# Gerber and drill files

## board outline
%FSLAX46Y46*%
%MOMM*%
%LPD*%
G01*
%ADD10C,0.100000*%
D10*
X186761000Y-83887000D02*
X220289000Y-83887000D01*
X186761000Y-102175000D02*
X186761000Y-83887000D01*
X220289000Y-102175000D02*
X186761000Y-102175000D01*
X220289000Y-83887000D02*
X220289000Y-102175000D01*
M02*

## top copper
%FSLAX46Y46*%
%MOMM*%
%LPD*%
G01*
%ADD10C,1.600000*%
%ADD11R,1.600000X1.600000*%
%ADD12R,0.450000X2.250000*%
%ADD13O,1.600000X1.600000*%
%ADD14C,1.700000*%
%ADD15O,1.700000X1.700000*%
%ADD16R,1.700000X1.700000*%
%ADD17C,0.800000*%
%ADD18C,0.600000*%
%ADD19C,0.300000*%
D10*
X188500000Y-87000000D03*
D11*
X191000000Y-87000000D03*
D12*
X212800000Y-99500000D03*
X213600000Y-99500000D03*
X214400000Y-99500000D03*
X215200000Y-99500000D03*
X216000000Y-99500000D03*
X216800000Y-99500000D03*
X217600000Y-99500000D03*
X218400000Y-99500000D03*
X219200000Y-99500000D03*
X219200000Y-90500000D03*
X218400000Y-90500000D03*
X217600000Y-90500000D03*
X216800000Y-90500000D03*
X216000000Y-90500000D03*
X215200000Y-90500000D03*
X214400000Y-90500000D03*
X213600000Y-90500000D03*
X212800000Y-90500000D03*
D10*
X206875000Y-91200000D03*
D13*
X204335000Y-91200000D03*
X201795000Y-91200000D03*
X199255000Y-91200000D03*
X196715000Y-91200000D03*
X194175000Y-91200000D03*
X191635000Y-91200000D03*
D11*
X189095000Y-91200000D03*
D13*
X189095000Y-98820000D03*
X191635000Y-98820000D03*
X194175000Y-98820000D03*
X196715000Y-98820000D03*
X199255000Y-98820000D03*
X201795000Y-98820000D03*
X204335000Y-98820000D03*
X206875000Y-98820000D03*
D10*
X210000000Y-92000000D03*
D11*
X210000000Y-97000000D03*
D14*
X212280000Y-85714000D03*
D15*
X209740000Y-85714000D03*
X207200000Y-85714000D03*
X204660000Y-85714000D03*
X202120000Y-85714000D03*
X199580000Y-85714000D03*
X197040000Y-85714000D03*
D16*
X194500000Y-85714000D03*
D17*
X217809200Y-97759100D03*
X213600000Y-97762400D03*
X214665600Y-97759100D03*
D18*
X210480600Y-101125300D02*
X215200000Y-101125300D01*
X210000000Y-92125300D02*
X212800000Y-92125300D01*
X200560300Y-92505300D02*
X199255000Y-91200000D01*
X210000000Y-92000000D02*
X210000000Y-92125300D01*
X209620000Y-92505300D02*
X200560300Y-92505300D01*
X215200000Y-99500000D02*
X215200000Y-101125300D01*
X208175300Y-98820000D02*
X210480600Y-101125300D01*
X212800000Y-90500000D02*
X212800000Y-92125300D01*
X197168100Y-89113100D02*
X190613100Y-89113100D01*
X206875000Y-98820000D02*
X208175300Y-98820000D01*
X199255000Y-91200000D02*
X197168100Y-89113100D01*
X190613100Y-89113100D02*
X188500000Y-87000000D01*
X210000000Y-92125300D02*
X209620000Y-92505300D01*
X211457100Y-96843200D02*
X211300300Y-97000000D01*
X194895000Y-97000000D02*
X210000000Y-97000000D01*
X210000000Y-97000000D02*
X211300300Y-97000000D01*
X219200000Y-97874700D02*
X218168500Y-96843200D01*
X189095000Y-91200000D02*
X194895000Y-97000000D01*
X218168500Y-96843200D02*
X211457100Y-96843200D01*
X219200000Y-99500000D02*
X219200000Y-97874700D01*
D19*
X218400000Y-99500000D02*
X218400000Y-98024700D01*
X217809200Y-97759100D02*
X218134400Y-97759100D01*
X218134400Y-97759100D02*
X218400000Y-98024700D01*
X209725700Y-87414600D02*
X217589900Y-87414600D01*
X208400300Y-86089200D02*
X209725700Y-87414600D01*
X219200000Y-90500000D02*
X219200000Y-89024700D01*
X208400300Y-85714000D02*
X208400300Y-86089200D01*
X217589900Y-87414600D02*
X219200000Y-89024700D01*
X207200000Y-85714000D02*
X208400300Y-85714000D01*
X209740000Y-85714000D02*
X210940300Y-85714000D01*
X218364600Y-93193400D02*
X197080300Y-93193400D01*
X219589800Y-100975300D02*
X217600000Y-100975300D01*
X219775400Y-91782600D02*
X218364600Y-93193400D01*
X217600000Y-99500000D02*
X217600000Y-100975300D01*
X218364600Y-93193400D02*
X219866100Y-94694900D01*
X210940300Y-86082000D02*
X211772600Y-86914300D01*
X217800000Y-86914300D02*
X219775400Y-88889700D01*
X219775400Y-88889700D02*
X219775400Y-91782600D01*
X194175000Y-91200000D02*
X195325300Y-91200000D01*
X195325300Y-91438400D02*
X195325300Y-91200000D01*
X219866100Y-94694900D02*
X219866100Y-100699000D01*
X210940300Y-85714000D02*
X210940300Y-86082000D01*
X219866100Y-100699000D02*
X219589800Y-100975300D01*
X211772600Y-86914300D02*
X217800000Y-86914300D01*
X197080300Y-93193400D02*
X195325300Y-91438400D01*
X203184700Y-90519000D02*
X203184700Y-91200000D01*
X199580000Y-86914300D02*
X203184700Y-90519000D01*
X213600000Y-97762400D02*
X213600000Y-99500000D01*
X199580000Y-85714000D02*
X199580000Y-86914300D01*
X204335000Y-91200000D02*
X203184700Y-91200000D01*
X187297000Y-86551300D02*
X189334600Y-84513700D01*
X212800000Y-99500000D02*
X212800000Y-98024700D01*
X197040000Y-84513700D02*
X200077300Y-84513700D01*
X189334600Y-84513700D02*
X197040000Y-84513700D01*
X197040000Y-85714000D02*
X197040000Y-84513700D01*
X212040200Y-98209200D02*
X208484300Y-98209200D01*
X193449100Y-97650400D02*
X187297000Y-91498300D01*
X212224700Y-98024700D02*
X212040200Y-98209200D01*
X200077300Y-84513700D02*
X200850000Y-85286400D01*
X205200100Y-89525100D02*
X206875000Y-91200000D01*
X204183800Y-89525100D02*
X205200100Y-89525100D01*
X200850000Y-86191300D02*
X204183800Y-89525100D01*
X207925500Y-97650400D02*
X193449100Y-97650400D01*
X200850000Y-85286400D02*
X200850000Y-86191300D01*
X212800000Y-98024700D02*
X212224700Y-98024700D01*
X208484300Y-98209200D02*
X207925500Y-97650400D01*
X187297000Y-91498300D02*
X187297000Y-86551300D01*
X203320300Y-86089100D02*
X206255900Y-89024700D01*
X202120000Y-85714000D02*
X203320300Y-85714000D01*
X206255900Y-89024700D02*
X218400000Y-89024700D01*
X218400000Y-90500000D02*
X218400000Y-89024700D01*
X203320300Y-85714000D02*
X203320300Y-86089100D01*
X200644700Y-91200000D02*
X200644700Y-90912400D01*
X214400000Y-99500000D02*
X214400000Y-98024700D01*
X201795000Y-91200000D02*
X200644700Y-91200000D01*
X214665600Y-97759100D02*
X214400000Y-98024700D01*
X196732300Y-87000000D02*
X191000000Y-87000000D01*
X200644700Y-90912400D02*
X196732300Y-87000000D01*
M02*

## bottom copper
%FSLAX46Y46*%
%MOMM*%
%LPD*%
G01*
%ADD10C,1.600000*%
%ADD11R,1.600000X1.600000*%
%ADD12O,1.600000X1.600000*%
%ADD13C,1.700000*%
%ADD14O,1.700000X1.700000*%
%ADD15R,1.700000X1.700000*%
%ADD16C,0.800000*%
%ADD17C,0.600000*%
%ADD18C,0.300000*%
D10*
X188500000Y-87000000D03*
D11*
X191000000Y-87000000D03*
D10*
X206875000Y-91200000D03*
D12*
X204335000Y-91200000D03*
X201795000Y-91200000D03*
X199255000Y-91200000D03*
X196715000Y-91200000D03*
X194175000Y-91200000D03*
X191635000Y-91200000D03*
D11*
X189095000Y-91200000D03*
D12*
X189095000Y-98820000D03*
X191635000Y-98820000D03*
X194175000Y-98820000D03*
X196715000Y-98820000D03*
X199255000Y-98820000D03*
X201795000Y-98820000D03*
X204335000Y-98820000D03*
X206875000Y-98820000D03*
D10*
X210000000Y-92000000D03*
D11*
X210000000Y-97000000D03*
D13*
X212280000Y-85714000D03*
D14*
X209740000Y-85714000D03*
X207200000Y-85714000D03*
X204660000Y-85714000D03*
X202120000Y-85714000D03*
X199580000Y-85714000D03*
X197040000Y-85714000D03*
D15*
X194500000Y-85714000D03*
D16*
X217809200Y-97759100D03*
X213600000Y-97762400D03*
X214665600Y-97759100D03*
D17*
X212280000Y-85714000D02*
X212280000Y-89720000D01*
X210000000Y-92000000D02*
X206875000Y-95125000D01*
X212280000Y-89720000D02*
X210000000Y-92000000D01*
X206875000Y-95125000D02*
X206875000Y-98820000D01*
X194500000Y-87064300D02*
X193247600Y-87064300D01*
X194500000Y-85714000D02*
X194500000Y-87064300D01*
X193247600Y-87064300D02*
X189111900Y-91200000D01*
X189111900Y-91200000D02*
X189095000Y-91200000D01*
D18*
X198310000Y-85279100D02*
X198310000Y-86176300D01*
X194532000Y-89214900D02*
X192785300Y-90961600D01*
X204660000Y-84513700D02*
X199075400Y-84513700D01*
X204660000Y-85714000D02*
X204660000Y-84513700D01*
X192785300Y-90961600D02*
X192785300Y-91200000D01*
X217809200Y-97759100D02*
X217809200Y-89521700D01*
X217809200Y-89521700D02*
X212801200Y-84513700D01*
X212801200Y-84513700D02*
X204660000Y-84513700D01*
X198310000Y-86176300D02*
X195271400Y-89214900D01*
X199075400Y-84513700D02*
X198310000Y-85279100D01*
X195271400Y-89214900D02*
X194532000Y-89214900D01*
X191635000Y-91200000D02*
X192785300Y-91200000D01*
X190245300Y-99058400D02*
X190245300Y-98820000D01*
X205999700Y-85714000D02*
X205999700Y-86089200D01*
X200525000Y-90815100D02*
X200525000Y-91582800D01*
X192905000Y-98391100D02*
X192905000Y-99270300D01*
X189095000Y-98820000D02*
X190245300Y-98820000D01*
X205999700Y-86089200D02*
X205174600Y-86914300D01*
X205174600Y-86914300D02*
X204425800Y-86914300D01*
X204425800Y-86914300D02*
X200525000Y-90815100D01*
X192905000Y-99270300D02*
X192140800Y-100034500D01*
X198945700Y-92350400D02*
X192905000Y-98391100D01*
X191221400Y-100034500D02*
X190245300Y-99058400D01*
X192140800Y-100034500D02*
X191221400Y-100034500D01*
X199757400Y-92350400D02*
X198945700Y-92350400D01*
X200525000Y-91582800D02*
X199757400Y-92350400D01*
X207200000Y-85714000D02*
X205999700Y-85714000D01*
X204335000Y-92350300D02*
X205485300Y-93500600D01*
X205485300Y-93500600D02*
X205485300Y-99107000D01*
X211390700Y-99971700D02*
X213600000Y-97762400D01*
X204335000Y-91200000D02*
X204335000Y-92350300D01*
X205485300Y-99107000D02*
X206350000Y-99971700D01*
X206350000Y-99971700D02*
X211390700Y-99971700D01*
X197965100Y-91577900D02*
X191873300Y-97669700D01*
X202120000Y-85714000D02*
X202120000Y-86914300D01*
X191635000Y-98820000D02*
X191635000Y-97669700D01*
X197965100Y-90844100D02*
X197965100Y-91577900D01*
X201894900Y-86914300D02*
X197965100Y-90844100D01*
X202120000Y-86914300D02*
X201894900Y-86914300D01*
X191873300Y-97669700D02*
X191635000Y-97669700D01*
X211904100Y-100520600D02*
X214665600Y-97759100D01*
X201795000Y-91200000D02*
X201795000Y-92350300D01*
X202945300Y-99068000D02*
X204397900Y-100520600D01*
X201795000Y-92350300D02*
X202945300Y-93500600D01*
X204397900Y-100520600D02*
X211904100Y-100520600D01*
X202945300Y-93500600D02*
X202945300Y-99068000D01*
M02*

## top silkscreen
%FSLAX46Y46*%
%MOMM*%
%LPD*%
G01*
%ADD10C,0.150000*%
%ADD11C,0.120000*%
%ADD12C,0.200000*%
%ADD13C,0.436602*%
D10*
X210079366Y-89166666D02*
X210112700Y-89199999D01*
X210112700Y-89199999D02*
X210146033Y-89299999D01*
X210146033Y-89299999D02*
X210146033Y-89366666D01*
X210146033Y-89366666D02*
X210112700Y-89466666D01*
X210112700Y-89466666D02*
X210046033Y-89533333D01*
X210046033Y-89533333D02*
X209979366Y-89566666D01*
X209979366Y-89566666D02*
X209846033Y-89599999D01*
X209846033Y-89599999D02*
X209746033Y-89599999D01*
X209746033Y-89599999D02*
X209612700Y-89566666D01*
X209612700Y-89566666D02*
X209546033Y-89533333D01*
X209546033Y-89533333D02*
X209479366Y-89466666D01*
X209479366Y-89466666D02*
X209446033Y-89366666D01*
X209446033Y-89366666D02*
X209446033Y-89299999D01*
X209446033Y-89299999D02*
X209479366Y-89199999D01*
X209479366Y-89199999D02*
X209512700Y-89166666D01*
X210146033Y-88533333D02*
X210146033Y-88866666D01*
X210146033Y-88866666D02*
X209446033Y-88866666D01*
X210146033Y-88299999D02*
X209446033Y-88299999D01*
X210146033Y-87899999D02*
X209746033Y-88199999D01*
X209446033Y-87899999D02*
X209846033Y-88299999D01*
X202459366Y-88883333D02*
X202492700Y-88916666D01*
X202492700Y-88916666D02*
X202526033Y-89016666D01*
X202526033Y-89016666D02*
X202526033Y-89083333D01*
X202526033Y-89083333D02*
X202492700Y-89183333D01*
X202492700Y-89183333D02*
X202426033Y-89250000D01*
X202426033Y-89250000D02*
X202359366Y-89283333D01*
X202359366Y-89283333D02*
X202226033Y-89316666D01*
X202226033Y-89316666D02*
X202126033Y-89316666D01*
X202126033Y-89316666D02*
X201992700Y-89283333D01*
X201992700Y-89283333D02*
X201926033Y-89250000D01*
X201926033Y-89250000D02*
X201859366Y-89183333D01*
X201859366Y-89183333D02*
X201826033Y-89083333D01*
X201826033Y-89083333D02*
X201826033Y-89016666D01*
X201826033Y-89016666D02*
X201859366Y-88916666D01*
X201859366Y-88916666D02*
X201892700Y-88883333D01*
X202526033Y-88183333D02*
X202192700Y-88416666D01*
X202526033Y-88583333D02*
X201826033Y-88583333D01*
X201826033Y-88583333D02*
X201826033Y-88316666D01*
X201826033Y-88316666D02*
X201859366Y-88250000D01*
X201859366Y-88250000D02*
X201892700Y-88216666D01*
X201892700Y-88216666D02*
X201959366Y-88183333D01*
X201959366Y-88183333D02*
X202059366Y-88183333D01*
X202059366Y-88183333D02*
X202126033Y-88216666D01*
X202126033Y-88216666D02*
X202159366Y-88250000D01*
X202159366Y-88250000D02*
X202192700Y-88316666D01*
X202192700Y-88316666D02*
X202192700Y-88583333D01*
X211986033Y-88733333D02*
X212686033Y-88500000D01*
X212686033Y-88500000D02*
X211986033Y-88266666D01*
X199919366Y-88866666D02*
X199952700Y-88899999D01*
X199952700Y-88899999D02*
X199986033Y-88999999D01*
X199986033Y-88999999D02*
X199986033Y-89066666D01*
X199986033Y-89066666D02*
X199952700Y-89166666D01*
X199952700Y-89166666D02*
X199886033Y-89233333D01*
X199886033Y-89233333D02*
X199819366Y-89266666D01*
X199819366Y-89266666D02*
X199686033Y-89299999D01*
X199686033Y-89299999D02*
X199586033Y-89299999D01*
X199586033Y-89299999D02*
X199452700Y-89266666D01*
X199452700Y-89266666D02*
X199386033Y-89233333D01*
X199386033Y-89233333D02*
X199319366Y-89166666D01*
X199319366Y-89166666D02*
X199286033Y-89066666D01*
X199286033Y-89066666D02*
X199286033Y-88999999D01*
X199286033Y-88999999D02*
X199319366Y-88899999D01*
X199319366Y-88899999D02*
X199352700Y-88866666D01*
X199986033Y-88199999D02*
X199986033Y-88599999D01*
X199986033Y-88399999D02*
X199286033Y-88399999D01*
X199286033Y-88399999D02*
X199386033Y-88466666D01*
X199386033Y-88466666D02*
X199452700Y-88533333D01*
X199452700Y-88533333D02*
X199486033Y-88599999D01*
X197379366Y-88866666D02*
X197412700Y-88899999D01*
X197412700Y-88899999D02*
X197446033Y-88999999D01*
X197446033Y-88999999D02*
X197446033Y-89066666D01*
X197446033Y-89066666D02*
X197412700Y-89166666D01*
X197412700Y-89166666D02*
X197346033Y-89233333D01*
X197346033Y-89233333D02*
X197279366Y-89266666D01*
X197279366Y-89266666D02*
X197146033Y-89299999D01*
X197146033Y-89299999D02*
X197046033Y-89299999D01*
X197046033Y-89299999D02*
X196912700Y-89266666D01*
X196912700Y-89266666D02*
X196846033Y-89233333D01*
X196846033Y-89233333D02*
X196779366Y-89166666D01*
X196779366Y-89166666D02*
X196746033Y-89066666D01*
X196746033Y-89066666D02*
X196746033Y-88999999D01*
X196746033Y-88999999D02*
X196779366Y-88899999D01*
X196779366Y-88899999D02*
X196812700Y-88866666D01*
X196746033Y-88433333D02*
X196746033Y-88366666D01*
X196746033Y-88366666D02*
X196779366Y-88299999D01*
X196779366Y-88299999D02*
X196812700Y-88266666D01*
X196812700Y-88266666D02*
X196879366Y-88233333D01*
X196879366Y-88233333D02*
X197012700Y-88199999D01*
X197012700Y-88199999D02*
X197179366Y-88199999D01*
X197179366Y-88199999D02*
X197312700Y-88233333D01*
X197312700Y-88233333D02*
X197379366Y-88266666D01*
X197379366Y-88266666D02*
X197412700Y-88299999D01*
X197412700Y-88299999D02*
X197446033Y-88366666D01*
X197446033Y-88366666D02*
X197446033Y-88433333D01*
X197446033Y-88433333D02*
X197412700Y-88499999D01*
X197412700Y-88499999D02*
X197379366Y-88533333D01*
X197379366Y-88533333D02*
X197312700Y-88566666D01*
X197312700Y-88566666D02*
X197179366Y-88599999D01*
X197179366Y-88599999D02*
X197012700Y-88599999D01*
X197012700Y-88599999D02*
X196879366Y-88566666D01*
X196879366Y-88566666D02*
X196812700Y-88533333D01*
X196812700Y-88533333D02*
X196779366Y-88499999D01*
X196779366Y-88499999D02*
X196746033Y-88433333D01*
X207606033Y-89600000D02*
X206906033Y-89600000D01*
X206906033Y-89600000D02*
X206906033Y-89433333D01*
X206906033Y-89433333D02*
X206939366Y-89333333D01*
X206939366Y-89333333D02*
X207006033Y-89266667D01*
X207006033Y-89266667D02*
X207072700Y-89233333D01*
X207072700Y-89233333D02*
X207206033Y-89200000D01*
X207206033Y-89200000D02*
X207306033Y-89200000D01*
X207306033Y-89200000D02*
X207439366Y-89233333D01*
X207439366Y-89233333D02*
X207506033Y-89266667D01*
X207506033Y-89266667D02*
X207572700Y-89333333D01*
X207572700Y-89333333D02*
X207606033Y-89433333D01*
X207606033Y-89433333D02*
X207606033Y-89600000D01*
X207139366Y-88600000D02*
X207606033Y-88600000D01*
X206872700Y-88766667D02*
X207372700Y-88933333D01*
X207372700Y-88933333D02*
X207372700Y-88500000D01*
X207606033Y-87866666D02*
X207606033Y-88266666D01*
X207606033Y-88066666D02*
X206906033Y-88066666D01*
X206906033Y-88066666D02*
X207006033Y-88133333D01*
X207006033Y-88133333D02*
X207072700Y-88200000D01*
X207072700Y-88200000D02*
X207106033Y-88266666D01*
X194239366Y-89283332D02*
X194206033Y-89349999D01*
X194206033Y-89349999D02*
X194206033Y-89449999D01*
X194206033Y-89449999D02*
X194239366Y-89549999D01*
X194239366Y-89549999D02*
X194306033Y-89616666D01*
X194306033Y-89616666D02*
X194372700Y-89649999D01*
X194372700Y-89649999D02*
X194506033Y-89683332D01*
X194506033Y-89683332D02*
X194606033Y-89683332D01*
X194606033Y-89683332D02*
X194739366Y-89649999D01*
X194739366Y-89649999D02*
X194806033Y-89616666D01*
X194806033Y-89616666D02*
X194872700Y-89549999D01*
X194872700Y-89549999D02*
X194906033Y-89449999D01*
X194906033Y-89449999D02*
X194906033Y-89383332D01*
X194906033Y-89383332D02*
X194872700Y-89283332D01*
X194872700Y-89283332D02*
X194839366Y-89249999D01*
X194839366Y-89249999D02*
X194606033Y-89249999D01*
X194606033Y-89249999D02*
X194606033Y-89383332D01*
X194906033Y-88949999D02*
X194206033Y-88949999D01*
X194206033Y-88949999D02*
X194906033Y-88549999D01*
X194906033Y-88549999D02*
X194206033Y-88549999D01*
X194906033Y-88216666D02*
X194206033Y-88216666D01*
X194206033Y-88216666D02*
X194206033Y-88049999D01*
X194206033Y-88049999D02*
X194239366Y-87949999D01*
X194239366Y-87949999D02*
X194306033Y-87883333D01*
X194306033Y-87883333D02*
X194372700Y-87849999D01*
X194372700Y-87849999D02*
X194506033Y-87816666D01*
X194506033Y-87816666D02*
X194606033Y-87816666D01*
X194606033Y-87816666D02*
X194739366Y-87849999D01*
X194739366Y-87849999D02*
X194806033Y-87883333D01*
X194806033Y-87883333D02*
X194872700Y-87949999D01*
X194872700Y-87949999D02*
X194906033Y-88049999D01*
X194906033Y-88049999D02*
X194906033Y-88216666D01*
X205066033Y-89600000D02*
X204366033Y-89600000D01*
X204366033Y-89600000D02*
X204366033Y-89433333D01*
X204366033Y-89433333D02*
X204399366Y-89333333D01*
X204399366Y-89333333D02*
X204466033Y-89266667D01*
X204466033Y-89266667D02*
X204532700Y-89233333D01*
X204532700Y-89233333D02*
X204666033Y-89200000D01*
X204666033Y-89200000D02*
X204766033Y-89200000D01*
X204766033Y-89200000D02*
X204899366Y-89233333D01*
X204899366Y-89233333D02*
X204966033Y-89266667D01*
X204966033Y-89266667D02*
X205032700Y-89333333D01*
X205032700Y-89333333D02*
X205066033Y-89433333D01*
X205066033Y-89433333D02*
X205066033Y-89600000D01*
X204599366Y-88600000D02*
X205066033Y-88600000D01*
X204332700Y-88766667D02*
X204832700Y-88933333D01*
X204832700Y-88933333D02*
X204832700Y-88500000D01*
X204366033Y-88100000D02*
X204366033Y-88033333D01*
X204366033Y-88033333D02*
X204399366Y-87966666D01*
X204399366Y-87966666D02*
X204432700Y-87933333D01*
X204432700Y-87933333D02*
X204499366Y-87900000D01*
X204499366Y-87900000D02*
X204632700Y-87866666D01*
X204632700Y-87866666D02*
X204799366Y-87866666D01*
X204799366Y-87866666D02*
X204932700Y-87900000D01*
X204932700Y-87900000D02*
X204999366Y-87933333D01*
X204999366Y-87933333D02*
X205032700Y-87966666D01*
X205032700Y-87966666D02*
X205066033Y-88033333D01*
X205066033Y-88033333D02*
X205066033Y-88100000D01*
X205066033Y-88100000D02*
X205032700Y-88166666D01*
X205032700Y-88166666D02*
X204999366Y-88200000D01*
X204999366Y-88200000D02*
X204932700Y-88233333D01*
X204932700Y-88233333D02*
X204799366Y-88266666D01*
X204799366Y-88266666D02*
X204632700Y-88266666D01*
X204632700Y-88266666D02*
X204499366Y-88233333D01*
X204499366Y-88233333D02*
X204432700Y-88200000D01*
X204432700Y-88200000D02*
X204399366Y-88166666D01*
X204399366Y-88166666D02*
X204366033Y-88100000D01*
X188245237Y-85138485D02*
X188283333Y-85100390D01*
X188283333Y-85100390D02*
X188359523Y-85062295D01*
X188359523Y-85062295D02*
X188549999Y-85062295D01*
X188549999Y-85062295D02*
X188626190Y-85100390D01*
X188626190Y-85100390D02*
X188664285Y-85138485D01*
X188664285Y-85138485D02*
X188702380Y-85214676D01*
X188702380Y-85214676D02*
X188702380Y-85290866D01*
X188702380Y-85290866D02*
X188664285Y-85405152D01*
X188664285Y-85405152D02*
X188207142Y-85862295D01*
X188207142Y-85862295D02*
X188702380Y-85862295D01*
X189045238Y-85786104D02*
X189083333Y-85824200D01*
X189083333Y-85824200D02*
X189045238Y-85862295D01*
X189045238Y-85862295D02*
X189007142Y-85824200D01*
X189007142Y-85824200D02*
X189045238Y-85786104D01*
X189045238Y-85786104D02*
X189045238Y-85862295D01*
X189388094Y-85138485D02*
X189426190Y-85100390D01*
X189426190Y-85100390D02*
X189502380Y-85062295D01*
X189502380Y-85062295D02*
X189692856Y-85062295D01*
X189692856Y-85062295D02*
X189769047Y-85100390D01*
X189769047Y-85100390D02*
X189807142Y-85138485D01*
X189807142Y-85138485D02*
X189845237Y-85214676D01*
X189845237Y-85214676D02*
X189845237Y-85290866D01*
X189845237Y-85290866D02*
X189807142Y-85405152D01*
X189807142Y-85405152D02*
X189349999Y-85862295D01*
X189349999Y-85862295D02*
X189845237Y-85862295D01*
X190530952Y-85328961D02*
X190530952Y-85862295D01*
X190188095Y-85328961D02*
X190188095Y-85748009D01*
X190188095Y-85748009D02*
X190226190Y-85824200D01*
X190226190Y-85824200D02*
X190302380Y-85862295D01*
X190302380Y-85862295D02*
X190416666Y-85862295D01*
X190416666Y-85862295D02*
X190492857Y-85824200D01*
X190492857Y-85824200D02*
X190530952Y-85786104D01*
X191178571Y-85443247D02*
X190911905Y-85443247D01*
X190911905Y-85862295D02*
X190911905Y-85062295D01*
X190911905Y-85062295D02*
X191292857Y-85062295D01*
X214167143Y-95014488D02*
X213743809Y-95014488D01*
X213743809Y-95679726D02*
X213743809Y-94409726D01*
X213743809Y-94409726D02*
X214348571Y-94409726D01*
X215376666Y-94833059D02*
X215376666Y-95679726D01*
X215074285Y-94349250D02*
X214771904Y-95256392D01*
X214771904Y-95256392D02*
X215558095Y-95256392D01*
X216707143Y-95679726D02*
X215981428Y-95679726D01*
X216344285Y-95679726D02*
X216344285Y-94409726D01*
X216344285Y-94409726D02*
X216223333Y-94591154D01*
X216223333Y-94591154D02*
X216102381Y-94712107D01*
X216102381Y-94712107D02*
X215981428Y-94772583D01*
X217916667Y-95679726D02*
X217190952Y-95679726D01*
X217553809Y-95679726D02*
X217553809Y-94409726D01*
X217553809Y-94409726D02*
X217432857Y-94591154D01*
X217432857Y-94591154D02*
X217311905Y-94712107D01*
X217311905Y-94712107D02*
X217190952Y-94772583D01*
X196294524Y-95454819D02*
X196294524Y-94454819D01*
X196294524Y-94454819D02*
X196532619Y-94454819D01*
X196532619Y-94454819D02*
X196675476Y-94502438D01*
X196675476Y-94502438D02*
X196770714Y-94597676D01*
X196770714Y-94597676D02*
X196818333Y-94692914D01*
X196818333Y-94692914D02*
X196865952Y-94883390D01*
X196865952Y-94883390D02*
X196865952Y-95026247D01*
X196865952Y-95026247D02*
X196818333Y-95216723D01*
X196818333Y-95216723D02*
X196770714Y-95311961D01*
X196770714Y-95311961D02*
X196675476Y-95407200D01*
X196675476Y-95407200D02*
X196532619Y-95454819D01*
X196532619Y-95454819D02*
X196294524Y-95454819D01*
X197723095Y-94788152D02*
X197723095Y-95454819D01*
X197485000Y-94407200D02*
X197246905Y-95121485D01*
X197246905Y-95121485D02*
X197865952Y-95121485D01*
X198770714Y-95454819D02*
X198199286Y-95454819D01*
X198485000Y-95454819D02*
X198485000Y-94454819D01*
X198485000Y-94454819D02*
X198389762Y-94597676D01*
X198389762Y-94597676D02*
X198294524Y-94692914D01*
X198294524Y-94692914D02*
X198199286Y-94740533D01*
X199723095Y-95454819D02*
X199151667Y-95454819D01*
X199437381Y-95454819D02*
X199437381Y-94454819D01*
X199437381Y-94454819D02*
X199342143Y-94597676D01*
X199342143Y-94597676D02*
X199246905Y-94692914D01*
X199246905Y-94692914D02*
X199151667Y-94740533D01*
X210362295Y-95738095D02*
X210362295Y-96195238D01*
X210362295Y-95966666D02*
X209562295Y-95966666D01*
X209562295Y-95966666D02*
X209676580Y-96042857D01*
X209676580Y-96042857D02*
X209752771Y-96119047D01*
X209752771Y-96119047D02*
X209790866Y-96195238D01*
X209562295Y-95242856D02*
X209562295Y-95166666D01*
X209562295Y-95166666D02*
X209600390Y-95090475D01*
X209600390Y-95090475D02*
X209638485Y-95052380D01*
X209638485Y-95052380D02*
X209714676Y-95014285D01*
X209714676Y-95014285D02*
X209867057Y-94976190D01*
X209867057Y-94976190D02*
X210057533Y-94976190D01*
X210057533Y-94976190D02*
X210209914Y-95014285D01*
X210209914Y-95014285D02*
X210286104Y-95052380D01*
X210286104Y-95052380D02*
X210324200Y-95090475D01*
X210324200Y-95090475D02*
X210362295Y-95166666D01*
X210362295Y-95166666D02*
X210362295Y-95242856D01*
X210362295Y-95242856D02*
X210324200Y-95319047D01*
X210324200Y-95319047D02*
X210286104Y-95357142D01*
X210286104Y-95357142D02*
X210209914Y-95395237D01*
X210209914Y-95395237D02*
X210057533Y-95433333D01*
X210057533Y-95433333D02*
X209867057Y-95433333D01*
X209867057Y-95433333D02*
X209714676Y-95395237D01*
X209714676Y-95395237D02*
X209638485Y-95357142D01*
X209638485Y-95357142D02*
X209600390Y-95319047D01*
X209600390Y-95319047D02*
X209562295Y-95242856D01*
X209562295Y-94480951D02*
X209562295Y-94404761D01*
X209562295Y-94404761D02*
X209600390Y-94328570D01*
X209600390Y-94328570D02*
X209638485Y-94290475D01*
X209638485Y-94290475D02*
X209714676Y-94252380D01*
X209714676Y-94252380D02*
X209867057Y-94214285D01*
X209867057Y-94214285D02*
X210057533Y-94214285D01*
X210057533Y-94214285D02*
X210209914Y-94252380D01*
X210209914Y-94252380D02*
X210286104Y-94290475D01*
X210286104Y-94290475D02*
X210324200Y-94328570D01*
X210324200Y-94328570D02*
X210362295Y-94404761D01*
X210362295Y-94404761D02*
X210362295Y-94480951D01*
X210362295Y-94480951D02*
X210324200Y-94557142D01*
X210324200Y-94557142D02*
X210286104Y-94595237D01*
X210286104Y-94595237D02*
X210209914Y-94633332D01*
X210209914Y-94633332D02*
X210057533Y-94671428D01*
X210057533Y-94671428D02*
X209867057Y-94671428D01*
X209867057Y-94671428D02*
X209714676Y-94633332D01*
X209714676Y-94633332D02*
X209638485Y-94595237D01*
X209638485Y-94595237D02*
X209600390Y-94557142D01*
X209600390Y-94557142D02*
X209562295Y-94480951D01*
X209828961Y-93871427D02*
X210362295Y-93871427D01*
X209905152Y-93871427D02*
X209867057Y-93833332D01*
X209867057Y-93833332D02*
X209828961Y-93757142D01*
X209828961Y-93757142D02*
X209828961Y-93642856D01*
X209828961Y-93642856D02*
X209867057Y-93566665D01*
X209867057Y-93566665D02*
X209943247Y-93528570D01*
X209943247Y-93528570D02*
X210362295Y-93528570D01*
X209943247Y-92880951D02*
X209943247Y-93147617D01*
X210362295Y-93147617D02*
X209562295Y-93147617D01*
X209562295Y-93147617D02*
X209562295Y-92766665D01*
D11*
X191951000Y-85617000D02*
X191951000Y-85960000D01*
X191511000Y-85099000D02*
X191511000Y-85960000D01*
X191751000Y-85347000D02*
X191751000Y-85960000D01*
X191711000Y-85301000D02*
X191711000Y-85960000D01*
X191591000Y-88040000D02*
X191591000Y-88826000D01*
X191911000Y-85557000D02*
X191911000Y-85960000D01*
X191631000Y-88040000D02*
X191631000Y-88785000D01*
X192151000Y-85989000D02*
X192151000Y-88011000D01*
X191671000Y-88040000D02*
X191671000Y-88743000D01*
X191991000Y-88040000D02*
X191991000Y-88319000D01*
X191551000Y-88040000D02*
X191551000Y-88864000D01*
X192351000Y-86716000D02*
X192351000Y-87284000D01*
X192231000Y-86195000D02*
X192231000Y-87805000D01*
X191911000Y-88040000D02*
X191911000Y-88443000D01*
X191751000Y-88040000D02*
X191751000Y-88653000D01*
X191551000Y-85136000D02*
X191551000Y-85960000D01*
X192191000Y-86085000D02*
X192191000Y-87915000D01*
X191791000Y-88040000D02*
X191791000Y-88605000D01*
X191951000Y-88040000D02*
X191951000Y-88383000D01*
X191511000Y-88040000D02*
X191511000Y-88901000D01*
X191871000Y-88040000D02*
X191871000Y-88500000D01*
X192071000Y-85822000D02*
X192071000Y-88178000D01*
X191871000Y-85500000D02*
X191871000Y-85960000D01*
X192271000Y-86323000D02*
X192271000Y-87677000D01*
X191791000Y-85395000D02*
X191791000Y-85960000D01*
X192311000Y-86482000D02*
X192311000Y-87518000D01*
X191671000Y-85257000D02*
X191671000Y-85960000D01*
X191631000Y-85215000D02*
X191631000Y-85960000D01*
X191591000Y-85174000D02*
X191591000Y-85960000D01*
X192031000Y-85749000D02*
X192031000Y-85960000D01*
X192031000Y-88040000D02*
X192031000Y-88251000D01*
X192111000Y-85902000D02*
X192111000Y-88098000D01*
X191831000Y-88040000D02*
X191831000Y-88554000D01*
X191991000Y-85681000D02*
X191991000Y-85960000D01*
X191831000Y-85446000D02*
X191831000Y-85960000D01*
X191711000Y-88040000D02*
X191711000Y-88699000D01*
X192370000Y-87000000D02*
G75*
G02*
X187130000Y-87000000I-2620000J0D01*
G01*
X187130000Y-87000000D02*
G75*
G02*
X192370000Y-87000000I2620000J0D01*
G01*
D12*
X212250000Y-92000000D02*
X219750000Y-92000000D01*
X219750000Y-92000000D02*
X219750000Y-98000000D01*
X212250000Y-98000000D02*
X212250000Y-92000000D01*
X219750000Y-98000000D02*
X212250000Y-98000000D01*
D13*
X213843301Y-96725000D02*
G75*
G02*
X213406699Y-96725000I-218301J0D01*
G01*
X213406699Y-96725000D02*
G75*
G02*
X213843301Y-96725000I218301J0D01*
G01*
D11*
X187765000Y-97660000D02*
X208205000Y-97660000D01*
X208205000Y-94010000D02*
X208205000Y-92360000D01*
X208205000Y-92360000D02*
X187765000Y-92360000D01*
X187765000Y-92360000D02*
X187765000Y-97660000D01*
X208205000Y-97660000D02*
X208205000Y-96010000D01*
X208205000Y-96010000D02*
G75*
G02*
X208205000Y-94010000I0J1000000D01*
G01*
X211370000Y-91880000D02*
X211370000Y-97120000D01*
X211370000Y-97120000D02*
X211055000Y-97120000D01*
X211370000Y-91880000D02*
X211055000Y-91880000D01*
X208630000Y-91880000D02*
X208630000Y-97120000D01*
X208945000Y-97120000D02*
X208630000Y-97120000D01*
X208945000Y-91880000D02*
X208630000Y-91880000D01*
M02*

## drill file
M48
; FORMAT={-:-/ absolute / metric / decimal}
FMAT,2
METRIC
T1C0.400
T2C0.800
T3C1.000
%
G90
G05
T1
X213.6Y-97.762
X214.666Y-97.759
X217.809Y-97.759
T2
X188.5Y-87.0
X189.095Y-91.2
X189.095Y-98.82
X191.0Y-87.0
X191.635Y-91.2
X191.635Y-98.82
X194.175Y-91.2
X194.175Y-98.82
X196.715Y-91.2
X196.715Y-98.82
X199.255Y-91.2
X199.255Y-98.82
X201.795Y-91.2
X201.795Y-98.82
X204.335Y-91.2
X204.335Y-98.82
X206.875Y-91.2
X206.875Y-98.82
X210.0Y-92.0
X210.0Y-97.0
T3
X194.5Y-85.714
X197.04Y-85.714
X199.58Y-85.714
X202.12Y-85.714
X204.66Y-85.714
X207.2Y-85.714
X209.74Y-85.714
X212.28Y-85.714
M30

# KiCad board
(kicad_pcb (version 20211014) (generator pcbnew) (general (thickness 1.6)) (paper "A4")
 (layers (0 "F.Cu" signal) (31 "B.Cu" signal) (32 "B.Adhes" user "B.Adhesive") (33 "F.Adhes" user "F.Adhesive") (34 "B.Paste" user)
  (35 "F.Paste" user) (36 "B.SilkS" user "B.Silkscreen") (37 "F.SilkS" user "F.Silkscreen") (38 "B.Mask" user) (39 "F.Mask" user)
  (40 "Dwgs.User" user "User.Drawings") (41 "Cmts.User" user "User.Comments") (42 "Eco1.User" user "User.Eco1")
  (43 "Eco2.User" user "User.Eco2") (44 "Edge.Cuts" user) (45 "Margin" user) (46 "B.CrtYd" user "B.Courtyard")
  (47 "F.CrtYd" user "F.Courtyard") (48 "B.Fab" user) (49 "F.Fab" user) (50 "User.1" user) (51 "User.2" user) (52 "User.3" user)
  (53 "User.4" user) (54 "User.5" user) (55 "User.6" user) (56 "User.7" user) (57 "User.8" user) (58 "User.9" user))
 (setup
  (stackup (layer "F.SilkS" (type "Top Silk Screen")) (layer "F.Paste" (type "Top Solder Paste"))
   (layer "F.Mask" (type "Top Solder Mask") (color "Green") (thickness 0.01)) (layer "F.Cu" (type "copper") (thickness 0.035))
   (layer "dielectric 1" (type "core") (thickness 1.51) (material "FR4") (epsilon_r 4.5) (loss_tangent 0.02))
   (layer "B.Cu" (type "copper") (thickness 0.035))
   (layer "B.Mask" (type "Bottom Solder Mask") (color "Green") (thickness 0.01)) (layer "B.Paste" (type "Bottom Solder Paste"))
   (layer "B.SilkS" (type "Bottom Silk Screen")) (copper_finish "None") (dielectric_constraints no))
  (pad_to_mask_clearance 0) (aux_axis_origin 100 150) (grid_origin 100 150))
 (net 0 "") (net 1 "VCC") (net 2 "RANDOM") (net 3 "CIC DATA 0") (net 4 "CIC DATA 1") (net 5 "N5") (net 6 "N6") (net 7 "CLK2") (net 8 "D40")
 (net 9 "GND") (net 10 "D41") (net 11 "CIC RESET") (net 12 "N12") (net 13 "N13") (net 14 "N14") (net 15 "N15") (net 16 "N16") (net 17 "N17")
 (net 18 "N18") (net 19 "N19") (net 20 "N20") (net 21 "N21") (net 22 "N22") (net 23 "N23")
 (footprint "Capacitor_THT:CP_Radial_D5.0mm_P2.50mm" (layer "F.Cu") (at 188.5 87)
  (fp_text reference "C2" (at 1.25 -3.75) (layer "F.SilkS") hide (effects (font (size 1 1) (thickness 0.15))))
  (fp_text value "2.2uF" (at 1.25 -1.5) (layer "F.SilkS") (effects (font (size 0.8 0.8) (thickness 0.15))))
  (fp_line (start 3.451 -1.383) (end 3.451 -1.04) (layer "F.SilkS") (width 0.12))
  (fp_line (start 3.011 -1.901) (end 3.011 -1.04) (layer "F.SilkS") (width 0.12))
  (fp_line (start 3.251 -1.653) (end 3.251 -1.04) (layer "F.SilkS") (width 0.12))
  (fp_line (start 3.211 -1.699) (end 3.211 -1.04) (layer "F.SilkS") (width 0.12))
  (fp_line (start 3.091 1.04) (end 3.091 1.826) (layer "F.SilkS") (width 0.12))
  (fp_line (start 3.411 -1.443) (end 3.411 -1.04) (layer "F.SilkS") (width 0.12))
  (fp_line (start 3.131 1.04) (end 3.131 1.785) (layer "F.SilkS") (width 0.12))
  (fp_line (start 3.651 -1.011) (end 3.651 1.011) (layer "F.SilkS") (width 0.12))
  (fp_line (start 3.171 1.04) (end 3.171 1.743) (layer "F.SilkS") (width 0.12))
  (fp_line (start 3.491 1.04) (end 3.491 1.319) (layer "F.SilkS") (width 0.12))
  (fp_line (start 3.051 1.04) (end 3.051 1.864) (layer "F.SilkS") (width 0.12))
  (fp_line (start 3.851 -0.284) (end 3.851 0.284) (layer "F.SilkS") (width 0.12))
  (fp_line (start 3.731 -0.805) (end 3.731 0.805) (layer "F.SilkS") (width 0.12))
  (fp_line (start 3.411 1.04) (end 3.411 1.443) (layer "F.SilkS") (width 0.12))
  (fp_line (start 3.251 1.04) (end 3.251 1.653) (layer "F.SilkS") (width 0.12))
  (fp_line (start 3.051 -1.864) (end 3.051 -1.04) (layer "F.SilkS") (width 0.12))
  (fp_line (start 3.691 -0.915) (end 3.691 0.915) (layer "F.SilkS") (width 0.12))
  (fp_line (start 3.291 1.04) (end 3.291 1.605) (layer "F.SilkS") (width 0.12))
  (fp_line (start 3.451 1.04) (end 3.451 1.383) (layer "F.SilkS") (width 0.12))
  (fp_line (start 3.011 1.04) (end 3.011 1.901) (layer "F.SilkS") (width 0.12))
  (fp_line (start 3.371 1.04) (end 3.371 1.5) (layer "F.SilkS") (width 0.12))
  (fp_line (start 3.571 -1.178) (end 3.571 1.178) (layer "F.SilkS") (width 0.12))
  (fp_line (start 3.371 -1.5) (end 3.371 -1.04) (layer "F.SilkS") (width 0.12))
  (fp_line (start 3.771 -0.677) (end 3.771 0.677) (layer "F.SilkS") (width 0.12))
  (fp_line (start 3.291 -1.605) (end 3.291 -1.04) (layer "F.SilkS") (width 0.12))
  (fp_line (start 3.811 -0.518) (end 3.811 0.518) (layer "F.SilkS") (width 0.12))
  (fp_line (start 3.171 -1.743) (end 3.171 -1.04) (layer "F.SilkS") (width 0.12))
  (fp_line (start 3.131 -1.785) (end 3.131 -1.04) (layer "F.SilkS") (width 0.12))
  (fp_line (start 3.091 -1.826) (end 3.091 -1.04) (layer "F.SilkS") (width 0.12))
  (fp_line (start 3.531 -1.251) (end 3.531 -1.04) (layer "F.SilkS") (width 0.12))
  (fp_line (start 3.531 1.04) (end 3.531 1.251) (layer "F.SilkS") (width 0.12))
  (fp_line (start 3.611 -1.098) (end 3.611 1.098) (layer "F.SilkS") (width 0.12))
  (fp_line (start 3.331 1.04) (end 3.331 1.554) (layer "F.SilkS") (width 0.12))
  (fp_line (start 3.491 -1.319) (end 3.491 -1.04) (layer "F.SilkS") (width 0.12))
  (fp_line (start 3.331 -1.554) (end 3.331 -1.04) (layer "F.SilkS") (width 0.12))
  (fp_line (start 3.211 1.04) (end 3.211 1.699) (layer "F.SilkS") (width 0.12))
  (fp_circle (center 1.25 0) (end 3.87 0) (layer "F.SilkS") (width 0.12) (fill none))
  (pad "1" thru_hole circle (at 0 0) (size 1.6 1.6) (drill 0.8) (layers *.Cu *.Mask) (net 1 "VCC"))
  (pad "2" thru_hole rect (at 2.5 0) (size 1.6 1.6) (drill 0.8) (layers *.Cu *.Mask) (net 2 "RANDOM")))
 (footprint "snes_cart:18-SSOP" (layer "F.Cu") (at 216 95 180)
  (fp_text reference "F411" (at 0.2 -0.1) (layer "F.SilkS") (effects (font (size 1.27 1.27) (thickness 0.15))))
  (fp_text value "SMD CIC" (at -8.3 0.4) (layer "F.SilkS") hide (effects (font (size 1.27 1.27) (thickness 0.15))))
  (fp_line (start 3.75 3) (end -3.75 3) (layer "F.SilkS") (width 0.2))
  (fp_line (start -3.75 3) (end -3.75 -3) (layer "F.SilkS") (width 0.2))
  (fp_line (start 3.75 -3) (end 3.75 3) (layer "F.SilkS") (width 0.2))
  (fp_line (start -3.75 -3) (end 3.75 -3) (layer "F.SilkS") (width 0.2))
  (fp_circle (center 2.375 -1.725) (end 2.593301 -1.725) (layer "F.SilkS") (width 0.436603) (fill solid))
  (pad "1" smd rect (at 3.2 -4.5 90) (size 2.25 0.45) (layers "F.Cu" "F.Paste" "F.Mask") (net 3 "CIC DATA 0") (solder_mask_margin 0.1016))
  (pad "2" smd rect (at 2.4 -4.5 90) (size 2.25 0.45) (layers "F.Cu" "F.Paste" "F.Mask") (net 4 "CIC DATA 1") (solder_mask_margin 0.1016))
  (pad "3" smd rect (at 1.6 -4.5 90) (size 2.25 0.45) (layers "F.Cu" "F.Paste" "F.Mask") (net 2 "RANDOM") (solder_mask_margin 0.1016))
  (pad "4" smd rect (at 0.8 -4.5 90) (size 2.25 0.45) (layers "F.Cu" "F.Paste" "F.Mask") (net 1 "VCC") (solder_mask_margin 0.1016))
  (pad "5" smd rect (at 0 -4.5 90) (size 2.25 0.45) (layers "F.Cu" "F.Paste" "F.Mask") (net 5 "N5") (solder_mask_margin 0.1016))
  (pad "6" smd rect (at -0.8 -4.5 90) (size 2.25 0.45) (layers "F.Cu" "F.Paste" "F.Mask") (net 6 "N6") (solder_mask_margin 0.1016))
  (pad "7" smd rect (at -1.6 -4.5 90) (size 2.25 0.45) (layers "F.Cu" "F.Paste" "F.Mask") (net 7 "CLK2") (solder_mask_margin 0.1016))
  (pad "8" smd rect (at -2.4 -4.5 90) (size 2.25 0.45) (layers "F.Cu" "F.Paste" "F.Mask") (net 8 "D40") (solder_mask_margin 0.1016))
  (pad "9" smd rect (at -3.2 -4.5 90) (size 2.25 0.45) (layers "F.Cu" "F.Paste" "F.Mask") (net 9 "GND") (solder_mask_margin 0.1016))
  (pad "10" smd rect (at -3.2 4.5 90) (size 2.25 0.45) (layers "F.Cu" "F.Paste" "F.Mask") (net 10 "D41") (solder_mask_margin 0.1016))
  (pad "11" smd rect (at -2.4 4.5 90) (size 2.25 0.45) (layers "F.Cu" "F.Paste" "F.Mask") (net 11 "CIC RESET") (solder_mask_margin 0.1016))
  (pad "12" smd rect (at -1.6 4.5 90) (size 2.25 0.45) (layers "F.Cu" "F.Paste" "F.Mask") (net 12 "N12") (solder_mask_margin 0.1016))
  (pad "13" smd rect (at -0.8 4.5 90) (size 2.25 0.45) (layers "F.Cu" "F.Paste" "F.Mask") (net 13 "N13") (solder_mask_margin 0.1016))
  (pad "14" smd rect (at 0 4.5 90) (size 2.25 0.45) (layers "F.Cu" "F.Paste" "F.Mask") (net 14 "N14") (solder_mask_margin 0.1016))
  (pad "15" smd rect (at 0.8 4.5 90) (size 2.25 0.45) (layers "F.Cu" "F.Paste" "F.Mask") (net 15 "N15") (solder_mask_margin 0.1016))
  (pad "16" smd rect (at 1.6 4.5 90) (size 2.25 0.45) (layers "F.Cu" "F.Paste" "F.Mask") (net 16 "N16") (solder_mask_margin 0.1016))
  (pad "17" smd rect (at 2.4 4.5 90) (size 2.25 0.45) (layers "F.Cu" "F.Paste" "F.Mask") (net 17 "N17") (solder_mask_margin 0.1016))
  (pad "18" smd rect (at 3.2 4.5 90) (size 2.25 0.45) (layers "F.Cu" "F.Paste" "F.Mask") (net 1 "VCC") (solder_mask_margin 0.1016)))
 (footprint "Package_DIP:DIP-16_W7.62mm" (layer "F.Cu") (at 206.875 91.2 -90)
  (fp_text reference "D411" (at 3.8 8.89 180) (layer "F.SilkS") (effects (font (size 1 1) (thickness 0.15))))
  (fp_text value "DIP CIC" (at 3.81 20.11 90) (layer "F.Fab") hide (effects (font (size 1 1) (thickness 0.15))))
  (fp_line (start 6.46 19.11) (end 6.46 -1.33) (layer "F.SilkS") (width 0.12))
  (fp_line (start 2.81 -1.33) (end 1.16 -1.33) (layer "F.SilkS") (width 0.12))
  (fp_line (start 1.16 -1.33) (end 1.16 19.11) (layer "F.SilkS") (width 0.12))
  (fp_line (start 1.16 19.11) (end 6.46 19.11) (layer "F.SilkS") (width 0.12))
  (fp_line (start 6.46 -1.33) (end 4.81 -1.33) (layer "F.SilkS") (width 0.12))
  (fp_arc (start 4.81 -1.33) (mid 3.81 -0.33) (end 2.81 -1.33) (layer "F.SilkS") (width 0.12))
  (pad "1" thru_hole circle (at 0 0 270) (size 1.6 1.6) (drill 0.8) (layers *.Cu *.Mask) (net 3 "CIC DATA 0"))
  (pad "2" thru_hole oval (at 0 2.54 270) (size 1.6 1.6) (drill 0.8) (layers *.Cu *.Mask) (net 4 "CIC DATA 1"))
  (pad "3" thru_hole oval (at 0 5.08 270) (size 1.6 1.6) (drill 0.8) (layers *.Cu *.Mask) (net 2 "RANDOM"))
  (pad "4" thru_hole oval (at 0 7.62 270) (size 1.6 1.6) (drill 0.8) (layers *.Cu *.Mask) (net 1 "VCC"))
  (pad "5" thru_hole oval (at 0 10.16 270) (size 1.6 1.6) (drill 0.8) (layers *.Cu *.Mask) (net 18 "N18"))
  (pad "6" thru_hole oval (at 0 12.7 270) (size 1.6 1.6) (drill 0.8) (layers *.Cu *.Mask) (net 7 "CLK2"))
  (pad "7" thru_hole oval (at 0 15.24 270) (size 1.6 1.6) (drill 0.8) (layers *.Cu *.Mask) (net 8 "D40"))
  (pad "8" thru_hole rect (at 0 17.78 270) (size 1.6 1.6) (drill 0.8) (layers *.Cu *.Mask) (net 9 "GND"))
  (pad "9" thru_hole oval (at 7.62 17.78 270) (size 1.6 1.6) (drill 0.8) (layers *.Cu *.Mask) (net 10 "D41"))
  (pad "10" thru_hole oval (at 7.62 15.24 270) (size 1.6 1.6) (drill 0.8) (layers *.Cu *.Mask) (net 11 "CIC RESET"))
  (pad "11" thru_hole oval (at 7.62 12.7 270) (size 1.6 1.6) (drill 0.8) (layers *.Cu *.Mask) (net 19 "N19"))
  (pad "12" thru_hole oval (at 7.62 10.16 270) (size 1.6 1.6) (drill 0.8) (layers *.Cu *.Mask) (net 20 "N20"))
  (pad "13" thru_hole oval (at 7.62 7.62 270) (size 1.6 1.6) (drill 0.8) (layers *.Cu *.Mask) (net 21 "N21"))
  (pad "14" thru_hole oval (at 7.62 5.08 270) (size 1.6 1.6) (drill 0.8) (layers *.Cu *.Mask) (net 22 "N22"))
  (pad "15" thru_hole oval (at 7.62 2.54 270) (size 1.6 1.6) (drill 0.8) (layers *.Cu *.Mask) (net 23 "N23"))
  (pad "16" thru_hole oval (at 7.62 0 270) (size 1.6 1.6) (drill 0.8) (layers *.Cu *.Mask) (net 1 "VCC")))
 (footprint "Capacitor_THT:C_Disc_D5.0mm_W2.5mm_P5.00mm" (layer "F.Cu") (at 210 92 -90)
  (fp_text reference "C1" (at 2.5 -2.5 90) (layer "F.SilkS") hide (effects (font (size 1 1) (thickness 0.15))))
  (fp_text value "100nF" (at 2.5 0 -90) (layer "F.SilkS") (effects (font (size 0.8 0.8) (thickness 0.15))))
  (fp_line (start -0.12 -1.37) (end 5.12 -1.37) (layer "F.SilkS") (width 0.12))
  (fp_line (start 5.12 -1.37) (end 5.12 -1.055) (layer "F.SilkS") (width 0.12))
  (fp_line (start -0.12 -1.37) (end -0.12 -1.055) (layer "F.SilkS") (width 0.12))
  (fp_line (start -0.12 1.37) (end 5.12 1.37) (layer "F.SilkS") (width 0.12))
  (fp_line (start 5.12 1.055) (end 5.12 1.37) (layer "F.SilkS") (width 0.12))
  (fp_line (start -0.12 1.055) (end -0.12 1.37) (layer "F.SilkS") (width 0.12))
  (pad "1" thru_hole circle (at 0 0 270) (size 1.6 1.6) (drill 0.8) (layers *.Cu *.Mask) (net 1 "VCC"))
  (pad "2" thru_hole rect (at 5 0 270) (size 1.6 1.6) (drill 0.8) (layers *.Cu *.Mask) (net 9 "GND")))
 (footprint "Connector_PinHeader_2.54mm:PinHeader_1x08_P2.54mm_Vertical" (layer "B.Cu") (at 212.28 85.714 90)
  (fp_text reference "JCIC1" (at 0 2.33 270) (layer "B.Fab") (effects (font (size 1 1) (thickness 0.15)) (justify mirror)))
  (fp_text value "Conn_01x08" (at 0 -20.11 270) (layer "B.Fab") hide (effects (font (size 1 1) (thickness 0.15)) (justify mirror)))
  (pad "1" thru_hole circle (at 0 0 90) (size 1.7 1.7) (drill 1) (layers *.Cu *.Mask) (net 1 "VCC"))
  (pad "2" thru_hole oval (at 0 -2.54 90) (size 1.7 1.7) (drill 1) (layers *.Cu *.Mask) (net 7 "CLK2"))
  (pad "3" thru_hole oval (at 0 -5.08 90) (size 1.7 1.7) (drill 1) (layers *.Cu *.Mask) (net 10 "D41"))
  (pad "4" thru_hole oval (at 0 -7.62 90) (size 1.7 1.7) (drill 1) (layers *.Cu *.Mask) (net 8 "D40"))
  (pad "5" thru_hole oval (at 0 -10.16 90) (size 1.7 1.7) (drill 1) (layers *.Cu *.Mask) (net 11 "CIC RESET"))
  (pad "6" thru_hole oval (at 0 -12.7 90) (size 1.7 1.7) (drill 1) (layers *.Cu *.Mask) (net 4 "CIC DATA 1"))
  (pad "7" thru_hole oval (at 0 -15.24 90) (size 1.7 1.7) (drill 1) (layers *.Cu *.Mask) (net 3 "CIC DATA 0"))
  (pad "8" thru_hole rect (at 0 -17.78 90) (size 1.7 1.7) (drill 1) (layers *.Cu *.Mask) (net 9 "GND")))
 (gr_line (start 186.761 83.887) (end 220.289 83.887) (layer "Edge.Cuts") (width 0.1))
 (gr_line (start 186.761 102.175) (end 186.761 83.887) (layer "Edge.Cuts") (width 0.1))
 (gr_line (start 220.289 102.175) (end 186.761 102.175) (layer "Edge.Cuts") (width 0.1))
 (gr_line (start 220.289 83.887) (end 220.289 102.175) (layer "Edge.Cuts") (width 0.1))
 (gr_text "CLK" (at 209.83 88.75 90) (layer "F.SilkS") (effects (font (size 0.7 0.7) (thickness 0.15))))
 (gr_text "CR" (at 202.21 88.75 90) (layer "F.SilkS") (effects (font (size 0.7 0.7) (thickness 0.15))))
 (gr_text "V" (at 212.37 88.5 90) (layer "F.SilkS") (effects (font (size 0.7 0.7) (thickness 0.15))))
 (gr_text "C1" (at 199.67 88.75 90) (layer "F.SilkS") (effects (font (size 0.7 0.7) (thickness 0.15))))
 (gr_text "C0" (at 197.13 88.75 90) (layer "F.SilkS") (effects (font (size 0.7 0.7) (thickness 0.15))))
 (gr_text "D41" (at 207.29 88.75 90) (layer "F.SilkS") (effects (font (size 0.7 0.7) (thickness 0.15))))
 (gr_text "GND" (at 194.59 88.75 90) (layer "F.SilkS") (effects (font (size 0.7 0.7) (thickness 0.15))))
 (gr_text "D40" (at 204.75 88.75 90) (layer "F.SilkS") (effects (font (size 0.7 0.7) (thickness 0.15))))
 (segment (start 210.4806 101.1253) (end 215.2 101.1253) (width 0.6) (layer "F.Cu") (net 1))
 (segment (start 210 92.1253) (end 212.8 92.1253) (width 0.6) (layer "F.Cu") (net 1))
 (segment (start 200.5603 92.5053) (end 199.255 91.2) (width 0.6) (layer "F.Cu") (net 1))
 (segment (start 210 92) (end 210 92.1253) (width 0.6) (layer "F.Cu") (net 1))
 (segment (start 209.62 92.5053) (end 200.5603 92.5053) (width 0.6) (layer "F.Cu") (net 1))
 (segment (start 215.2 99.5) (end 215.2 101.1253) (width 0.6) (layer "F.Cu") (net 1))
 (segment (start 208.1753 98.82) (end 210.4806 101.1253) (width 0.6) (layer "F.Cu") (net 1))
 (segment (start 212.8 90.5) (end 212.8 92.1253) (width 0.6) (layer "F.Cu") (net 1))
 (segment (start 197.1681 89.1131) (end 190.6131 89.1131) (width 0.6) (layer "F.Cu") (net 1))
 (segment (start 206.875 98.82) (end 208.1753 98.82) (width 0.6) (layer "F.Cu") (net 1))
 (segment (start 199.255 91.2) (end 197.1681 89.1131) (width 0.6) (layer "F.Cu") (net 1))
 (segment (start 190.6131 89.1131) (end 188.5 87) (width 0.6) (layer "F.Cu") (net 1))
 (segment (start 210 92.1253) (end 209.62 92.5053) (width 0.6) (layer "F.Cu") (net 1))
 (segment (start 212.28 85.714) (end 212.28 89.72) (width 0.6) (layer "B.Cu") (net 1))
 (segment (start 210 92) (end 206.875 95.125) (width 0.6) (layer "B.Cu") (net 1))
 (segment (start 212.28 89.72) (end 210 92) (width 0.6) (layer "B.Cu") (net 1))
 (segment (start 206.875 95.125) (end 206.875 98.82) (width 0.6) (layer "B.Cu") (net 1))
 (segment (start 211.4571 96.8432) (end 211.3003 97) (width 0.6) (layer "F.Cu") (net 9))
 (segment (start 194.895 97) (end 210 97) (width 0.6) (layer "F.Cu") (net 9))
 (segment (start 210 97) (end 211.3003 97) (width 0.6) (layer "F.Cu") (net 9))
 (segment (start 219.2 97.8747) (end 218.1685 96.8432) (width 0.6) (layer "F.Cu") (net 9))
 (segment (start 189.095 91.2) (end 194.895 97) (width 0.6) (layer "F.Cu") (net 9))
 (segment (start 218.1685 96.8432) (end 211.4571 96.8432) (width 0.6) (layer "F.Cu") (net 9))
 (segment (start 219.2 99.5) (end 219.2 97.8747) (width 0.6) (layer "F.Cu") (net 9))
 (segment (start 194.5 87.0643) (end 193.2476 87.0643) (width 0.6) (layer "B.Cu") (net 9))
 (segment (start 194.5 85.714) (end 194.5 87.0643) (width 0.6) (layer "B.Cu") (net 9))
 (segment (start 193.2476 87.0643) (end 189.1119 91.2) (width 0.6) (layer "B.Cu") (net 9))
 (segment (start 189.1119 91.2) (end 189.095 91.2) (width 0.6) (layer "B.Cu") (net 9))
 (segment (start 218.4 99.5) (end 218.4 98.0247) (width 0.3) (layer "F.Cu") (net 8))
 (segment (start 217.8092 97.7591) (end 218.1344 97.7591) (width 0.3) (layer "F.Cu") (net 8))
 (segment (start 218.1344 97.7591) (end 218.4 98.0247) (width 0.3) (layer "F.Cu") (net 8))
 (via (at 217.8092 97.7591) (size 0.8) (drill 0.4) (layers "F.Cu" "B.Cu") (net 8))
 (segment (start 198.31 85.2791) (end 198.31 86.1763) (width 0.3) (layer "B.Cu") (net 8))
 (segment (start 194.532 89.2149) (end 192.7853 90.9616) (width 0.3) (layer "B.Cu") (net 8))
 (segment (start 204.66 84.5137) (end 199.0754 84.5137) (width 0.3) (layer "B.Cu") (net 8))
 (segment (start 204.66 85.714) (end 204.66 84.5137) (width 0.3) (layer "B.Cu") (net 8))
 (segment (start 192.7853 90.9616) (end 192.7853 91.2) (width 0.3) (layer "B.Cu") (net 8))
 (segment (start 217.8092 97.7591) (end 217.8092 89.5217) (width 0.3) (layer "B.Cu") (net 8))
 (segment (start 217.8092 89.5217) (end 212.8012 84.5137) (width 0.3) (layer "B.Cu") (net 8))
 (segment (start 212.8012 84.5137) (end 204.66 84.5137) (width 0.3) (layer "B.Cu") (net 8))
 (segment (start 198.31 86.1763) (end 195.2714 89.2149) (width 0.3) (layer "B.Cu") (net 8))
 (segment (start 199.0754 84.5137) (end 198.31 85.2791) (width 0.3) (layer "B.Cu") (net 8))
 (segment (start 195.2714 89.2149) (end 194.532 89.2149) (width 0.3) (layer "B.Cu") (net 8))
 (segment (start 191.635 91.2) (end 192.7853 91.2) (width 0.3) (layer "B.Cu") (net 8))
 (segment (start 209.7257 87.4146) (end 217.5899 87.4146) (width 0.3) (layer "F.Cu") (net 10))
 (segment (start 208.4003 86.0892) (end 209.7257 87.4146) (width 0.3) (layer "F.Cu") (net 10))
 (segment (start 219.2 90.5) (end 219.2 89.0247) (width 0.3) (layer "F.Cu") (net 10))
 (segment (start 208.4003 85.714) (end 208.4003 86.0892) (width 0.3) (layer "F.Cu") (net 10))
 (segment (start 217.5899 87.4146) (end 219.2 89.0247) (width 0.3) (layer "F.Cu") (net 10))
 (segment (start 207.2 85.714) (end 208.4003 85.714) (width 0.3) (layer "F.Cu") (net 10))
 (segment (start 190.2453 99.0584) (end 190.2453 98.82) (width 0.3) (layer "B.Cu") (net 10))
 (segment (start 205.9997 85.714) (end 205.9997 86.0892) (width 0.3) (layer "B.Cu") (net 10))
 (segment (start 200.525 90.8151) (end 200.525 91.5828) (width 0.3) (layer "B.Cu") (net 10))
 (segment (start 192.905 98.3911) (end 192.905 99.2703) (width 0.3) (layer "B.Cu") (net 10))
 (segment (start 189.095 98.82) (end 190.2453 98.82) (width 0.3) (layer "B.Cu") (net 10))
 (segment (start 205.9997 86.0892) (end 205.1746 86.9143) (width 0.3) (layer "B.Cu") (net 10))
 (segment (start 205.1746 86.9143) (end 204.4258 86.9143) (width 0.3) (layer "B.Cu") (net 10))
 (segment (start 204.4258 86.9143) (end 200.525 90.8151) (width 0.3) (layer "B.Cu") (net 10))
 (segment (start 192.905 99.2703) (end 192.1408 100.0345) (width 0.3) (layer "B.Cu") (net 10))
 (segment (start 198.9457 92.3504) (end 192.905 98.3911) (width 0.3) (layer "B.Cu") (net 10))
 (segment (start 191.2214 100.0345) (end 190.2453 99.0584) (width 0.3) (layer "B.Cu") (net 10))
 (segment (start 192.1408 100.0345) (end 191.2214 100.0345) (width 0.3) (layer "B.Cu") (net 10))
 (segment (start 199.7574 92.3504) (end 198.9457 92.3504) (width 0.3) (layer "B.Cu") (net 10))
 (segment (start 200.525 91.5828) (end 199.7574 92.3504) (width 0.3) (layer "B.Cu") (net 10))
 (segment (start 207.2 85.714) (end 205.9997 85.714) (width 0.3) (layer "B.Cu") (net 10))
 (segment (start 209.74 85.714) (end 210.9403 85.714) (width 0.3) (layer "F.Cu") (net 7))
 (segment (start 218.3646 93.1934) (end 197.0803 93.1934) (width 0.3) (layer "F.Cu") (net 7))
 (segment (start 219.5898 100.9753) (end 217.6 100.9753) (width 0.3) (layer "F.Cu") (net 7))
 (segment (start 219.7754 91.7826) (end 218.3646 93.1934) (width 0.3) (layer "F.Cu") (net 7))
 (segment (start 217.6 99.5) (end 217.6 100.9753) (width 0.3) (layer "F.Cu") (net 7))
 (segment (start 218.3646 93.1934) (end 219.8661 94.6949) (width 0.3) (layer "F.Cu") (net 7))
 (segment (start 210.9403 86.082) (end 211.7726 86.9143) (width 0.3) (layer "F.Cu") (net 7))
 (segment (start 217.8 86.9143) (end 219.7754 88.8897) (width 0.3) (layer "F.Cu") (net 7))
 (segment (start 219.7754 88.8897) (end 219.7754 91.7826) (width 0.3) (layer "F.Cu") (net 7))
 (segment (start 194.175 91.2) (end 195.3253 91.2) (width 0.3) (layer "F.Cu") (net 7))
 (segment (start 195.3253 91.4384) (end 195.3253 91.2) (width 0.3) (layer "F.Cu") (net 7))
 (segment (start 219.8661 94.6949) (end 219.8661 100.699) (width 0.3) (layer "F.Cu") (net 7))
 (segment (start 210.9403 85.714) (end 210.9403 86.082) (width 0.3) (layer "F.Cu") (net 7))
 (segment (start 219.8661 100.699) (end 219.5898 100.9753) (width 0.3) (layer "F.Cu") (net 7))
 (segment (start 211.7726 86.9143) (end 217.8 86.9143) (width 0.3) (layer "F.Cu") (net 7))
 (segment (start 197.0803 93.1934) (end 195.3253 91.4384) (width 0.3) (layer "F.Cu") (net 7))
 (segment (start 203.1847 90.519) (end 203.1847 91.2) (width 0.3) (layer "F.Cu") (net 4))
 (segment (start 199.58 86.9143) (end 203.1847 90.519) (width 0.3) (layer "F.Cu") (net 4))
 (segment (start 213.6 97.7624) (end 213.6 99.5) (width 0.3) (layer "F.Cu") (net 4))
 (segment (start 199.58 85.714) (end 199.58 86.9143) (width 0.3) (layer "F.Cu") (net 4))
 (segment (start 204.335 91.2) (end 203.1847 91.2) (width 0.3) (layer "F.Cu") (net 4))
 (via (at 213.6 97.7624) (size 0.8) (drill 0.4) (layers "F.Cu" "B.Cu") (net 4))
 (segment (start 204.335 92.3503) (end 205.4853 93.5006) (width 0.3) (layer "B.Cu") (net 4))
 (segment (start 205.4853 93.5006) (end 205.4853 99.107) (width 0.3) (layer "B.Cu") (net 4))
 (segment (start 211.3907 99.9717) (end 213.6 97.7624) (width 0.3) (layer "B.Cu") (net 4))
 (segment (start 204.335 91.2) (end 204.335 92.3503) (width 0.3) (layer "B.Cu") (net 4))
 (segment (start 205.4853 99.107) (end 206.35 99.9717) (width 0.3) (layer "B.Cu") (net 4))
 (segment (start 206.35 99.9717) (end 211.3907 99.9717) (width 0.3) (layer "B.Cu") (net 4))
 (segment (start 187.297 86.5513) (end 189.3346 84.5137) (width 0.3) (layer "F.Cu") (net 3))
 (segment (start 212.8 99.5) (end 212.8 98.0247) (width 0.3) (layer "F.Cu") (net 3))
 (segment (start 197.04 84.5137) (end 200.0773 84.5137) (width 0.3) (layer "F.Cu") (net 3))
 (segment (start 189.3346 84.5137) (end 197.04 84.5137) (width 0.3) (layer "F.Cu") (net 3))
 (segment (start 197.04 85.714) (end 197.04 84.5137) (width 0.3) (layer "F.Cu") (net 3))
 (segment (start 212.0402 98.2092) (end 208.4843 98.2092) (width 0.3) (layer "F.Cu") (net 3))
 (segment (start 193.4491 97.6504) (end 187.297 91.4983) (width 0.3) (layer "F.Cu") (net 3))
 (segment (start 212.2247 98.0247) (end 212.0402 98.2092) (width 0.3) (layer "F.Cu") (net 3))
 (segment (start 200.0773 84.5137) (end 200.85 85.2864) (width 0.3) (layer "F.Cu") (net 3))
 (segment (start 205.2001 89.5251) (end 206.875 91.2) (width 0.3) (layer "F.Cu") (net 3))
 (segment (start 204.1838 89.5251) (end 205.2001 89.5251) (width 0.3) (layer "F.Cu") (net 3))
 (segment (start 200.85 86.1913) (end 204.1838 89.5251) (width 0.3) (layer "F.Cu") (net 3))
 (segment (start 207.9255 97.6504) (end 193.4491 97.6504) (width 0.3) (layer "F.Cu") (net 3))
 (segment (start 200.85 85.2864) (end 200.85 86.1913) (width 0.3) (layer "F.Cu") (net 3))
 (segment (start 212.8 98.0247) (end 212.2247 98.0247) (width 0.3) (layer "F.Cu") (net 3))
 (segment (start 208.4843 98.2092) (end 207.9255 97.6504) (width 0.3) (layer "F.Cu") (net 3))
 (segment (start 187.297 91.4983) (end 187.297 86.5513) (width 0.3) (layer "F.Cu") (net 3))
 (segment (start 203.3203 86.0891) (end 206.2559 89.0247) (width 0.3) (layer "F.Cu") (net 11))
 (segment (start 202.12 85.714) (end 203.3203 85.714) (width 0.3) (layer "F.Cu") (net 11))
 (segment (start 206.2559 89.0247) (end 218.4 89.0247) (width 0.3) (layer "F.Cu") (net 11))
 (segment (start 218.4 90.5) (end 218.4 89.0247) (width 0.3) (layer "F.Cu") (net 11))
 (segment (start 203.3203 85.714) (end 203.3203 86.0891) (width 0.3) (layer "F.Cu") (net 11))
 (segment (start 197.9651 91.5779) (end 191.8733 97.6697) (width 0.3) (layer "B.Cu") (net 11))
 (segment (start 202.12 85.714) (end 202.12 86.9143) (width 0.3) (layer "B.Cu") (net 11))
 (segment (start 191.635 98.82) (end 191.635 97.6697) (width 0.3) (layer "B.Cu") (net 11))
 (segment (start 197.9651 90.8441) (end 197.9651 91.5779) (width 0.3) (layer "B.Cu") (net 11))
 (segment (start 201.8949 86.9143) (end 197.9651 90.8441) (width 0.3) (layer "B.Cu") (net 11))
 (segment (start 202.12 86.9143) (end 201.8949 86.9143) (width 0.3) (layer "B.Cu") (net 11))
 (segment (start 191.8733 97.6697) (end 191.635 97.6697) (width 0.3) (layer "B.Cu") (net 11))
 (segment (start 200.6447 91.2) (end 200.6447 90.9124) (width 0.3) (layer "F.Cu") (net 2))
 (segment (start 214.4 99.5) (end 214.4 98.0247) (width 0.3) (layer "F.Cu") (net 2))
 (segment (start 201.795 91.2) (end 200.6447 91.2) (width 0.3) (layer "F.Cu") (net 2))
 (segment (start 214.6656 97.7591) (end 214.4 98.0247) (width 0.3) (layer "F.Cu") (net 2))
 (segment (start 196.7323 87) (end 191 87) (width 0.3) (layer "F.Cu") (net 2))
 (segment (start 200.6447 90.9124) (end 196.7323 87) (width 0.3) (layer "F.Cu") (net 2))
 (via (at 214.6656 97.7591) (size 0.8) (drill 0.4) (layers "F.Cu" "B.Cu") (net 2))
 (segment (start 211.9041 100.5206) (end 214.6656 97.7591) (width 0.3) (layer "B.Cu") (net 2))
 (segment (start 201.795 91.2) (end 201.795 92.3503) (width 0.3) (layer "B.Cu") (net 2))
 (segment (start 202.9453 99.068) (end 204.3979 100.5206) (width 0.3) (layer "B.Cu") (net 2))
 (segment (start 201.795 92.3503) (end 202.9453 93.5006) (width 0.3) (layer "B.Cu") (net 2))
 (segment (start 204.3979 100.5206) (end 211.9041 100.5206) (width 0.3) (layer "B.Cu") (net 2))
 (segment (start 202.9453 93.5006) (end 202.9453 99.068) (width 0.3) (layer "B.Cu") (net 2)))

